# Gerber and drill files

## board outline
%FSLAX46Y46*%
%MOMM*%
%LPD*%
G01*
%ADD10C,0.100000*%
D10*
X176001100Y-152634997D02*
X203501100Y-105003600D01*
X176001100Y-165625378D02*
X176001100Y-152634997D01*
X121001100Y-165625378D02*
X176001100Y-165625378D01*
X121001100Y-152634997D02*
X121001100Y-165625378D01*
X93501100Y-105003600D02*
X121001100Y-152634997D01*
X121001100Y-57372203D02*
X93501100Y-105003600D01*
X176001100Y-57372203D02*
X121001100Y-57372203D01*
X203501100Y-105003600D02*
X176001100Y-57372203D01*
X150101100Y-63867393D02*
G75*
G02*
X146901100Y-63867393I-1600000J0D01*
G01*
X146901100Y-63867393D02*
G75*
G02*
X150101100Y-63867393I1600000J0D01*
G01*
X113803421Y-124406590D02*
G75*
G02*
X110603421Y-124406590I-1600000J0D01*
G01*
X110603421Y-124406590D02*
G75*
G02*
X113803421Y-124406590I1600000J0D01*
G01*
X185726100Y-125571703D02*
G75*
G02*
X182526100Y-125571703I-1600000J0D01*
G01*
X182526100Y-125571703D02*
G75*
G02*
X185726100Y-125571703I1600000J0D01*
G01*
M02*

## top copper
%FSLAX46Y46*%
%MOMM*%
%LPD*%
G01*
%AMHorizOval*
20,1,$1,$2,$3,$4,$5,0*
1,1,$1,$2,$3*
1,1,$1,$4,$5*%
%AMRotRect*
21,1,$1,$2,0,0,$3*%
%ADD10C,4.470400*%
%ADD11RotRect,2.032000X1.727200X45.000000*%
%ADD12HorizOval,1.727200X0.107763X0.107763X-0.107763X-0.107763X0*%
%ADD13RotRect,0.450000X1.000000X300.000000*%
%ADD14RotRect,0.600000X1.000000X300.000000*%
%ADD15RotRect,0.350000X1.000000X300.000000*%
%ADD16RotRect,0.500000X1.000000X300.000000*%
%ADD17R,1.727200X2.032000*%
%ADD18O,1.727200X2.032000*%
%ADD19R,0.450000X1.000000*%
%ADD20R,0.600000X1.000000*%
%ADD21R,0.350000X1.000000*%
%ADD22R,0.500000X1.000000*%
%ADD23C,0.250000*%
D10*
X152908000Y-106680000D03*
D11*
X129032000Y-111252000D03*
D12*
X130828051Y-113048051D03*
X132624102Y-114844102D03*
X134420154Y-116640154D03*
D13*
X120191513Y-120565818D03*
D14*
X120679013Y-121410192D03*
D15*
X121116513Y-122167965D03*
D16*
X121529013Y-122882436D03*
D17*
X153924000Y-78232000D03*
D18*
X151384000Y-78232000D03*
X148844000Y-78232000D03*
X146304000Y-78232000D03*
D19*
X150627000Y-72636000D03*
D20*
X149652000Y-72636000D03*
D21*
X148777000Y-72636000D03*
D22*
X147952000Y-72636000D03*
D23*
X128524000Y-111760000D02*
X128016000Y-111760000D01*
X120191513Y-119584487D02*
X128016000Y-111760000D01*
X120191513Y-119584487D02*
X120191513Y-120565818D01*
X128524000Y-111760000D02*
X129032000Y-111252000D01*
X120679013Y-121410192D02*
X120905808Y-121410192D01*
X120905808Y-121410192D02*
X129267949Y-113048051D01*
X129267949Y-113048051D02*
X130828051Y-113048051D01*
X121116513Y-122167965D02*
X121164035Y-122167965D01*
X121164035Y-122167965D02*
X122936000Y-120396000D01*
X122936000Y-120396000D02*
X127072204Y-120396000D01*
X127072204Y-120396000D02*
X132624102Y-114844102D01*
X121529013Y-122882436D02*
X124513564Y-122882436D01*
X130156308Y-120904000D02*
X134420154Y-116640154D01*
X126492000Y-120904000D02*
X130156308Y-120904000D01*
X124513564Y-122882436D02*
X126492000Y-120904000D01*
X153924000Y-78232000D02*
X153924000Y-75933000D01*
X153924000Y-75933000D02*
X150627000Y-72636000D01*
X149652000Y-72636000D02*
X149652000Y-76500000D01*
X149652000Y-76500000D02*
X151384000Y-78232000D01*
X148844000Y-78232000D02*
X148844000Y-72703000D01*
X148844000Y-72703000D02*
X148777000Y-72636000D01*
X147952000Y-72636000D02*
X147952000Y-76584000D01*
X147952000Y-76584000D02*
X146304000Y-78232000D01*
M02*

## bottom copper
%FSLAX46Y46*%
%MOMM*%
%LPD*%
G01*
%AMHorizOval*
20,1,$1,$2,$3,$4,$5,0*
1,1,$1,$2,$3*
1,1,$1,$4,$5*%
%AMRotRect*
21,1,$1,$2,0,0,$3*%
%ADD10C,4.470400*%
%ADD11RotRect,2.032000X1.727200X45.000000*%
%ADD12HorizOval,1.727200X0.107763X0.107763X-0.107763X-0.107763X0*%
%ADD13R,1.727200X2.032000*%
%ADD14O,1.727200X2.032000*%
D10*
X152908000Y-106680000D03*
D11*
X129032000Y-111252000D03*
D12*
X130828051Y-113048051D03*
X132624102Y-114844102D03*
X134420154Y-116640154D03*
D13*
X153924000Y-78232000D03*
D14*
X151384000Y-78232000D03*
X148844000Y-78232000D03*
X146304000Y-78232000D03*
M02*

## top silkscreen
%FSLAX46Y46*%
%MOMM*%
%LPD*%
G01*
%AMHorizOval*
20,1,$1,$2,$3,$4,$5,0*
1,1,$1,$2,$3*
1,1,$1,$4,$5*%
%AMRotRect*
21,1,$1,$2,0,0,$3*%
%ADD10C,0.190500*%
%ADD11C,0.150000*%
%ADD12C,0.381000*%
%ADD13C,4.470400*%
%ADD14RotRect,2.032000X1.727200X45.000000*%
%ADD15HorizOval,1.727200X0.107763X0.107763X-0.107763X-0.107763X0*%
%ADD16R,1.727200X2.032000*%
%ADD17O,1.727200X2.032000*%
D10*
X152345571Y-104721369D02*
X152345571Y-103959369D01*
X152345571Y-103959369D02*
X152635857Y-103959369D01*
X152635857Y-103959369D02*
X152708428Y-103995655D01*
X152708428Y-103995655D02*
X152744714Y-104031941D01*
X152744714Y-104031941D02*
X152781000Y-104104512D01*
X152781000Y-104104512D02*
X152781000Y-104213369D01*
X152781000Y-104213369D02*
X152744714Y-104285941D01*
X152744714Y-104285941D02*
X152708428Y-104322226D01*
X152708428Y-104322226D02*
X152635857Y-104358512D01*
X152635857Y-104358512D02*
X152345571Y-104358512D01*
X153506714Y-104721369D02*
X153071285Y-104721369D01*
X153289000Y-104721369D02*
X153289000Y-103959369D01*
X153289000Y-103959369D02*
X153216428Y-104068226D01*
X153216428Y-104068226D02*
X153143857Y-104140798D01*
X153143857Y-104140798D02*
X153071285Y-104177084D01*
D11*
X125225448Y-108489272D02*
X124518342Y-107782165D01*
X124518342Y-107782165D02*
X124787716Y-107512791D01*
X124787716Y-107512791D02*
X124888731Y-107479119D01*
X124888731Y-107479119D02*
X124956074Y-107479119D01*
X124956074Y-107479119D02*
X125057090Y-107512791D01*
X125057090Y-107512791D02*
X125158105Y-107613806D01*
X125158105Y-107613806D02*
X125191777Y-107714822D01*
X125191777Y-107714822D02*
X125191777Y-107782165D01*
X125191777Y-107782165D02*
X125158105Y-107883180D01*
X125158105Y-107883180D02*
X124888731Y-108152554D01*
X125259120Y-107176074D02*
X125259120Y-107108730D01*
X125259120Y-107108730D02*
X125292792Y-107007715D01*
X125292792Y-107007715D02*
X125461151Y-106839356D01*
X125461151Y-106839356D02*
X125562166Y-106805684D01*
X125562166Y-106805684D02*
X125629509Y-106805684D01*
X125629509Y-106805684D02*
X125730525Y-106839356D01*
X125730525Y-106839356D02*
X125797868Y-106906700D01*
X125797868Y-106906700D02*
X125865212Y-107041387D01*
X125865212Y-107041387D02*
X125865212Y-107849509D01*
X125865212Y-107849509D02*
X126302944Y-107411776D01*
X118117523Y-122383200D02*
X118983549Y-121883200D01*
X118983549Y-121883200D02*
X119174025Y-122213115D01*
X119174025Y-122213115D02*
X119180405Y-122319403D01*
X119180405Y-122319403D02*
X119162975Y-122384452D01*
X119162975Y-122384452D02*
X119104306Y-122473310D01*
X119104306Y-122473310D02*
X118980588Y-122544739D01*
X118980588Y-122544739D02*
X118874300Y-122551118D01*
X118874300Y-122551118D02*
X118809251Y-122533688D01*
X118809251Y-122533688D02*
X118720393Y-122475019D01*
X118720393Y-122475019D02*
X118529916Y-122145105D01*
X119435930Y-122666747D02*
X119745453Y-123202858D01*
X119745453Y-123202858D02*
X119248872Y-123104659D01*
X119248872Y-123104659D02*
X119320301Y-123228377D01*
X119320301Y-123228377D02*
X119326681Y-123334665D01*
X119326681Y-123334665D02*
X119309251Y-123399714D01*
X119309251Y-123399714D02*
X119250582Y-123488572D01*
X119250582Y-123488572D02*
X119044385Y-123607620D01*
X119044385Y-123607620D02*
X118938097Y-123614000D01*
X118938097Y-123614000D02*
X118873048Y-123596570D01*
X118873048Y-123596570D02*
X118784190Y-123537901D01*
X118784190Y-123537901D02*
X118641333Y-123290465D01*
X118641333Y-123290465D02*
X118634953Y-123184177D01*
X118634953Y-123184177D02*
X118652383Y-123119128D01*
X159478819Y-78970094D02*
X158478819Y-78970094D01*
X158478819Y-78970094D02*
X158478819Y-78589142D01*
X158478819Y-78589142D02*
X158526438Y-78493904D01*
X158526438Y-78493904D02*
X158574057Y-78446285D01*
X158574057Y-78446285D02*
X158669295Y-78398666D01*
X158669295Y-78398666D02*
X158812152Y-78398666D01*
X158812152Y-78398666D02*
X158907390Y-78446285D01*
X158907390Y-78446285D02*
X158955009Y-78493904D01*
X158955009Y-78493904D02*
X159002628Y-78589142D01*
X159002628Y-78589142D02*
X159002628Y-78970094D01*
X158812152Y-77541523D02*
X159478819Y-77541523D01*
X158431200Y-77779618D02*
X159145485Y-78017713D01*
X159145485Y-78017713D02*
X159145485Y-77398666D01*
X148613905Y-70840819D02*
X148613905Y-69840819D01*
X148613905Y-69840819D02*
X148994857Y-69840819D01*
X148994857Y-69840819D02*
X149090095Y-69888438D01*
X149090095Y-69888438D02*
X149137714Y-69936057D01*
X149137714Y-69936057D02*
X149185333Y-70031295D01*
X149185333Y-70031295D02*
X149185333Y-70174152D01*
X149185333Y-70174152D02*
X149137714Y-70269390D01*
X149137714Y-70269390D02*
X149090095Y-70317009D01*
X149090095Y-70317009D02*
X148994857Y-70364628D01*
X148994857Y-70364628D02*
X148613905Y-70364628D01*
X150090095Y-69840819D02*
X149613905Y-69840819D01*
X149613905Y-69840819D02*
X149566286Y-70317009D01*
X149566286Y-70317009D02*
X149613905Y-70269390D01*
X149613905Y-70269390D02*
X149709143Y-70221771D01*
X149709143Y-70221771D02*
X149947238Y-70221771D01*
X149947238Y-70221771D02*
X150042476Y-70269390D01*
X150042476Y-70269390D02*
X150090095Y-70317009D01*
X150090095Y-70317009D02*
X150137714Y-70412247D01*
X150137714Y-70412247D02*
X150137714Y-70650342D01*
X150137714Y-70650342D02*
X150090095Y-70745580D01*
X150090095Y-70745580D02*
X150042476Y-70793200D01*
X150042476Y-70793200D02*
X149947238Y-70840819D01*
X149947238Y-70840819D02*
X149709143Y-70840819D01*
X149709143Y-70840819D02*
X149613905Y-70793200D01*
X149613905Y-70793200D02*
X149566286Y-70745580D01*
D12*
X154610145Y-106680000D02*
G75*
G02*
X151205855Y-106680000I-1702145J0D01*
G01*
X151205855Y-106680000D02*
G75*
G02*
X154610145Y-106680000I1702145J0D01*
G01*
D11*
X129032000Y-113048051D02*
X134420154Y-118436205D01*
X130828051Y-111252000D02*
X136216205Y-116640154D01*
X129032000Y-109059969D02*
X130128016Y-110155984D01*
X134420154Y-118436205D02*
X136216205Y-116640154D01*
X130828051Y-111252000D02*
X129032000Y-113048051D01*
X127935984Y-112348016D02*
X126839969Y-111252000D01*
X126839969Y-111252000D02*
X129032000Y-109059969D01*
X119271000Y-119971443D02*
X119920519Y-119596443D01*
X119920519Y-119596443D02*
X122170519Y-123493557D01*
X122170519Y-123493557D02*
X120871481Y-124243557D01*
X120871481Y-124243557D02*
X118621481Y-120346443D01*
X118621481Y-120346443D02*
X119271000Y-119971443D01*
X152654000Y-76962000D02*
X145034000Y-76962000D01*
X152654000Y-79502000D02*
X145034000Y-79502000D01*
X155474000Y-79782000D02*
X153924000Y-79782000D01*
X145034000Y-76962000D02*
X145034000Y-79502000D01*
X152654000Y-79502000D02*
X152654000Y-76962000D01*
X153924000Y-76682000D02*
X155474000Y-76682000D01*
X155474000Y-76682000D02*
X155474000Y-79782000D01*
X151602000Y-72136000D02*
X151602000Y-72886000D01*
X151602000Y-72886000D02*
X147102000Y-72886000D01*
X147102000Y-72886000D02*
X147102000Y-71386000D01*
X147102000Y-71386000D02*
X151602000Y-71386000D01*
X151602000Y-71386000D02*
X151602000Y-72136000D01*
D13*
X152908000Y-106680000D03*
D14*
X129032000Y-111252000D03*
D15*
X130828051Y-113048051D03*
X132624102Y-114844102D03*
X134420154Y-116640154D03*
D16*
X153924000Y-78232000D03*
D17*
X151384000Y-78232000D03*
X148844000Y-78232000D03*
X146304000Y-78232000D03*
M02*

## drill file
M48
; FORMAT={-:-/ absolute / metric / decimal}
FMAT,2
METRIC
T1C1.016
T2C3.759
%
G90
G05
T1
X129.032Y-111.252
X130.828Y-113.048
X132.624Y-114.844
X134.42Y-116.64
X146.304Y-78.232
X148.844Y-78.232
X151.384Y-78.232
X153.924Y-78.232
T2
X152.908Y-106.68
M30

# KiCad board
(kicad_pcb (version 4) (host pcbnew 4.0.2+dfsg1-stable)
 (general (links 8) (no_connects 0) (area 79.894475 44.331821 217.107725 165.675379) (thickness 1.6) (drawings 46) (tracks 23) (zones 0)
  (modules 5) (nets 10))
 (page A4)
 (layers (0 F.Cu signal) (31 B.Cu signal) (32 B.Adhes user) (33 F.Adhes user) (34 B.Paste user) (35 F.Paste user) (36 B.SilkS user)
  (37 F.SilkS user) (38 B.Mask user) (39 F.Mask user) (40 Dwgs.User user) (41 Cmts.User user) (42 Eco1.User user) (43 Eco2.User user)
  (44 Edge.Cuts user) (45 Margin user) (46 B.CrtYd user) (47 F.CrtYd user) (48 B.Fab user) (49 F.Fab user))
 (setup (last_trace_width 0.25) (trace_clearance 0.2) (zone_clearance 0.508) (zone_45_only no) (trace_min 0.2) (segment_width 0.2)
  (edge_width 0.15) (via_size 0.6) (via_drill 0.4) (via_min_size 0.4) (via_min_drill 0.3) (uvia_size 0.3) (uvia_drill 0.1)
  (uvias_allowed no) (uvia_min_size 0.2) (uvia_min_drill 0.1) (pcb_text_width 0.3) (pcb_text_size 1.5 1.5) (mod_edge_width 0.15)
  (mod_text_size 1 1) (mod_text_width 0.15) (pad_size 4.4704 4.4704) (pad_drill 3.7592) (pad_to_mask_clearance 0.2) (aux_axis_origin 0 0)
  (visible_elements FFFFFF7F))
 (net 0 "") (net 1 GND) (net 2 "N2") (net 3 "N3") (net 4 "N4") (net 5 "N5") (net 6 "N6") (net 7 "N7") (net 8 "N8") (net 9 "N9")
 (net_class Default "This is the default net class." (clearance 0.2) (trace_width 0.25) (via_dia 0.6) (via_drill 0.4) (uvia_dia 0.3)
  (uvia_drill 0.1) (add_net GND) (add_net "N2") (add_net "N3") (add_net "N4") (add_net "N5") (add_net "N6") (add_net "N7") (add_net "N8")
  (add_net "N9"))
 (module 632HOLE (layer F.Cu) (at 152.908 106.68)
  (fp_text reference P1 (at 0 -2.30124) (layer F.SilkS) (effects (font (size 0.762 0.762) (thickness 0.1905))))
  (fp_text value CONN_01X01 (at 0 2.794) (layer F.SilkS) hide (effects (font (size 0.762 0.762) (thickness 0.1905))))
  (fp_circle (center 0 0) (end 1.69926 -0.09906) (layer F.SilkS) (width 0.381))
  (pad 1 thru_hole circle (at 0 0) (size 4.4704 4.4704) (drill 3.7592) (layers *.Cu *.Mask F.SilkS) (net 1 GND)))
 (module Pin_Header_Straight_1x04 (layer F.Cu) (at 129.032 111.252 45)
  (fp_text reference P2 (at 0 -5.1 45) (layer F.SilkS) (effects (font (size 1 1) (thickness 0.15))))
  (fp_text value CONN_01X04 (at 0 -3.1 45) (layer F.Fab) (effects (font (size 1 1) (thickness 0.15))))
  (fp_line (start -1.27 1.27) (end -1.27 8.89) (layer F.SilkS) (width 0.15))
  (fp_line (start 1.27 1.27) (end 1.27 8.89) (layer F.SilkS) (width 0.15))
  (fp_line (start 1.55 -1.55) (end 1.55 0) (layer F.SilkS) (width 0.15))
  (fp_line (start -1.27 8.89) (end 1.27 8.89) (layer F.SilkS) (width 0.15))
  (fp_line (start 1.27 1.27) (end -1.27 1.27) (layer F.SilkS) (width 0.15))
  (fp_line (start -1.55 0) (end -1.55 -1.55) (layer F.SilkS) (width 0.15))
  (fp_line (start -1.55 -1.55) (end 1.55 -1.55) (layer F.SilkS) (width 0.15))
  (pad 1 thru_hole rect (at 0 0 45) (size 2.032 1.7272) (drill 1.016) (layers *.Cu *.Mask F.SilkS) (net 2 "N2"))
  (pad 2 thru_hole oval (at 0 2.54 45) (size 2.032 1.7272) (drill 1.016) (layers *.Cu *.Mask F.SilkS) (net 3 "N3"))
  (pad 3 thru_hole oval (at 0 5.08 45) (size 2.032 1.7272) (drill 1.016) (layers *.Cu *.Mask F.SilkS) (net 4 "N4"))
  (pad 4 thru_hole oval (at 0 7.62 45) (size 2.032 1.7272) (drill 1.016) (layers *.Cu *.Mask F.SilkS) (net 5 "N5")))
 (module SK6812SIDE (layer F.Cu) (at 120.396 121.92 300)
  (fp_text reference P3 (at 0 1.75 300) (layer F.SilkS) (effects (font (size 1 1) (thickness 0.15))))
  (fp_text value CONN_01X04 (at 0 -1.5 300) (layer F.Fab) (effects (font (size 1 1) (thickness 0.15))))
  (fp_line (start -2.25 0) (end -2.25 -0.75) (layer F.SilkS) (width 0.15))
  (fp_line (start -2.25 -0.75) (end 2.25 -0.75) (layer F.SilkS) (width 0.15))
  (fp_line (start 2.25 -0.75) (end 2.25 0.75) (layer F.SilkS) (width 0.15))
  (fp_line (start 2.25 0.75) (end -2.25 0.75) (layer F.SilkS) (width 0.15))
  (fp_line (start -2.25 0.75) (end -2.25 0) (layer F.SilkS) (width 0.15))
  (pad 1 smd rect (at -1.275 -0.5 300) (size 0.45 1) (layers F.Cu F.Paste F.Mask) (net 2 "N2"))
  (pad 2 smd rect (at -0.3 -0.5 300) (size 0.6 1) (layers F.Cu F.Paste F.Mask) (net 3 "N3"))
  (pad 3 smd rect (at 0.575 -0.5 300) (size 0.35 1) (layers F.Cu F.Paste F.Mask) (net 4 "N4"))
  (pad 4 smd rect (at 1.4 -0.5 300) (size 0.5 1) (layers F.Cu F.Paste F.Mask) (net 5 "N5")))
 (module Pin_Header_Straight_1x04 (layer F.Cu) (at 153.924 78.232 270)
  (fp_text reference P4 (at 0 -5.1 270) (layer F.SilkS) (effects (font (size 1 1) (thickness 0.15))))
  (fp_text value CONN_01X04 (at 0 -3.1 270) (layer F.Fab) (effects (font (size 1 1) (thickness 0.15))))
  (fp_line (start -1.27 1.27) (end -1.27 8.89) (layer F.SilkS) (width 0.15))
  (fp_line (start 1.27 1.27) (end 1.27 8.89) (layer F.SilkS) (width 0.15))
  (fp_line (start 1.55 -1.55) (end 1.55 0) (layer F.SilkS) (width 0.15))
  (fp_line (start -1.27 8.89) (end 1.27 8.89) (layer F.SilkS) (width 0.15))
  (fp_line (start 1.27 1.27) (end -1.27 1.27) (layer F.SilkS) (width 0.15))
  (fp_line (start -1.55 0) (end -1.55 -1.55) (layer F.SilkS) (width 0.15))
  (fp_line (start -1.55 -1.55) (end 1.55 -1.55) (layer F.SilkS) (width 0.15))
  (pad 1 thru_hole rect (at 0 0 270) (size 2.032 1.7272) (drill 1.016) (layers *.Cu *.Mask F.SilkS) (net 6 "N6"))
  (pad 2 thru_hole oval (at 0 2.54 270) (size 2.032 1.7272) (drill 1.016) (layers *.Cu *.Mask F.SilkS) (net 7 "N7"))
  (pad 3 thru_hole oval (at 0 5.08 270) (size 2.032 1.7272) (drill 1.016) (layers *.Cu *.Mask F.SilkS) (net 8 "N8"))
  (pad 4 thru_hole oval (at 0 7.62 270) (size 2.032 1.7272) (drill 1.016) (layers *.Cu *.Mask F.SilkS) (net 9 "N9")))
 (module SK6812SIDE (layer F.Cu) (at 149.352 72.136 180)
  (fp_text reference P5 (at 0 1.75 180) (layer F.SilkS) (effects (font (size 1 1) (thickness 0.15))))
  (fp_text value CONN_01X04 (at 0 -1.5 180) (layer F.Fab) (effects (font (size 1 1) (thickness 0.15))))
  (fp_line (start -2.25 0) (end -2.25 -0.75) (layer F.SilkS) (width 0.15))
  (fp_line (start -2.25 -0.75) (end 2.25 -0.75) (layer F.SilkS) (width 0.15))
  (fp_line (start 2.25 -0.75) (end 2.25 0.75) (layer F.SilkS) (width 0.15))
  (fp_line (start 2.25 0.75) (end -2.25 0.75) (layer F.SilkS) (width 0.15))
  (fp_line (start -2.25 0.75) (end -2.25 0) (layer F.SilkS) (width 0.15))
  (pad 1 smd rect (at -1.275 -0.5 180) (size 0.45 1) (layers F.Cu F.Paste F.Mask) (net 6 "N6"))
  (pad 2 smd rect (at -0.3 -0.5 180) (size 0.6 1) (layers F.Cu F.Paste F.Mask) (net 7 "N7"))
  (pad 3 smd rect (at 0.575 -0.5 180) (size 0.35 1) (layers F.Cu F.Paste F.Mask) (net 8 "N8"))
  (pad 4 smd rect (at 1.4 -0.5 180) (size 0.5 1) (layers F.Cu F.Paste F.Mask) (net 9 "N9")))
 (gr_line (start 176.0011 152.634997) (end 203.5011 105.0036) (layer Edge.Cuts) (width 0.1))
 (gr_line (start 176.0011 165.625378) (end 176.0011 152.634997) (layer Edge.Cuts) (width 0.1))
 (gr_line (start 121.0011 165.625378) (end 176.0011 165.625378) (layer Edge.Cuts) (width 0.1))
 (gr_line (start 121.0011 152.634997) (end 121.0011 165.625378) (layer Edge.Cuts) (width 0.1))
 (gr_line (start 93.5011 105.0036) (end 121.0011 152.634997) (layer Edge.Cuts) (width 0.1))
 (gr_line (start 121.0011 57.372203) (end 93.5011 105.0036) (layer Edge.Cuts) (width 0.1))
 (gr_line (start 176.0011 57.372203) (end 121.0011 57.372203) (layer Edge.Cuts) (width 0.1))
 (gr_line (start 203.5011 105.0036) (end 176.0011 57.372203) (layer Edge.Cuts) (width 0.1))
 (gr_circle (center 148.5011 63.867393) (end 150.1011 63.867393) (layer Edge.Cuts) (width 0.1))
 (gr_circle (center 112.203421 124.40659) (end 113.803421 124.40659) (layer Edge.Cuts) (width 0.1))
 (gr_circle (center 184.1261 125.571703) (end 185.7261 125.571703) (layer Edge.Cuts) (width 0.1))
 (segment (start 128.524 111.76) (end 128.016 111.76) (width 0.25) (layer F.Cu) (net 2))
 (segment (start 120.191513 119.584487) (end 128.016 111.76) (width 0.25) (layer F.Cu) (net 2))
 (segment (start 120.191513 119.584487) (end 120.191513 120.565818) (width 0.25) (layer F.Cu) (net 2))
 (segment (start 128.524 111.76) (end 129.032 111.252) (width 0.25) (layer F.Cu) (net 2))
 (segment (start 120.679013 121.410192) (end 120.905808 121.410192) (width 0.25) (layer F.Cu) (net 3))
 (segment (start 120.905808 121.410192) (end 129.267949 113.048051) (width 0.25) (layer F.Cu) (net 3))
 (segment (start 129.267949 113.048051) (end 130.828051 113.048051) (width 0.25) (layer F.Cu) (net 3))
 (segment (start 121.116513 122.167965) (end 121.164035 122.167965) (width 0.25) (layer F.Cu) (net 4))
 (segment (start 121.164035 122.167965) (end 122.936 120.396) (width 0.25) (layer F.Cu) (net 4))
 (segment (start 122.936 120.396) (end 127.072204 120.396) (width 0.25) (layer F.Cu) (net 4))
 (segment (start 127.072204 120.396) (end 132.624102 114.844102) (width 0.25) (layer F.Cu) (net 4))
 (segment (start 121.529013 122.882436) (end 124.513564 122.882436) (width 0.25) (layer F.Cu) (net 5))
 (segment (start 130.156308 120.904) (end 134.420154 116.640154) (width 0.25) (layer F.Cu) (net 5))
 (segment (start 126.492 120.904) (end 130.156308 120.904) (width 0.25) (layer F.Cu) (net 5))
 (segment (start 124.513564 122.882436) (end 126.492 120.904) (width 0.25) (layer F.Cu) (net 5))
 (segment (start 153.924 78.232) (end 153.924 75.933) (width 0.25) (layer F.Cu) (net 6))
 (segment (start 153.924 75.933) (end 150.627 72.636) (width 0.25) (layer F.Cu) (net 6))
 (segment (start 149.652 72.636) (end 149.652 76.5) (width 0.25) (layer F.Cu) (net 7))
 (segment (start 149.652 76.5) (end 151.384 78.232) (width 0.25) (layer F.Cu) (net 7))
 (segment (start 148.844 78.232) (end 148.844 72.703) (width 0.25) (layer F.Cu) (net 8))
 (segment (start 148.844 72.703) (end 148.777 72.636) (width 0.25) (layer F.Cu) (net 8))
 (segment (start 147.952 72.636) (end 147.952 76.584) (width 0.25) (layer F.Cu) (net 9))
 (segment (start 147.952 76.584) (end 146.304 78.232) (width 0.25) (layer F.Cu) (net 9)))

